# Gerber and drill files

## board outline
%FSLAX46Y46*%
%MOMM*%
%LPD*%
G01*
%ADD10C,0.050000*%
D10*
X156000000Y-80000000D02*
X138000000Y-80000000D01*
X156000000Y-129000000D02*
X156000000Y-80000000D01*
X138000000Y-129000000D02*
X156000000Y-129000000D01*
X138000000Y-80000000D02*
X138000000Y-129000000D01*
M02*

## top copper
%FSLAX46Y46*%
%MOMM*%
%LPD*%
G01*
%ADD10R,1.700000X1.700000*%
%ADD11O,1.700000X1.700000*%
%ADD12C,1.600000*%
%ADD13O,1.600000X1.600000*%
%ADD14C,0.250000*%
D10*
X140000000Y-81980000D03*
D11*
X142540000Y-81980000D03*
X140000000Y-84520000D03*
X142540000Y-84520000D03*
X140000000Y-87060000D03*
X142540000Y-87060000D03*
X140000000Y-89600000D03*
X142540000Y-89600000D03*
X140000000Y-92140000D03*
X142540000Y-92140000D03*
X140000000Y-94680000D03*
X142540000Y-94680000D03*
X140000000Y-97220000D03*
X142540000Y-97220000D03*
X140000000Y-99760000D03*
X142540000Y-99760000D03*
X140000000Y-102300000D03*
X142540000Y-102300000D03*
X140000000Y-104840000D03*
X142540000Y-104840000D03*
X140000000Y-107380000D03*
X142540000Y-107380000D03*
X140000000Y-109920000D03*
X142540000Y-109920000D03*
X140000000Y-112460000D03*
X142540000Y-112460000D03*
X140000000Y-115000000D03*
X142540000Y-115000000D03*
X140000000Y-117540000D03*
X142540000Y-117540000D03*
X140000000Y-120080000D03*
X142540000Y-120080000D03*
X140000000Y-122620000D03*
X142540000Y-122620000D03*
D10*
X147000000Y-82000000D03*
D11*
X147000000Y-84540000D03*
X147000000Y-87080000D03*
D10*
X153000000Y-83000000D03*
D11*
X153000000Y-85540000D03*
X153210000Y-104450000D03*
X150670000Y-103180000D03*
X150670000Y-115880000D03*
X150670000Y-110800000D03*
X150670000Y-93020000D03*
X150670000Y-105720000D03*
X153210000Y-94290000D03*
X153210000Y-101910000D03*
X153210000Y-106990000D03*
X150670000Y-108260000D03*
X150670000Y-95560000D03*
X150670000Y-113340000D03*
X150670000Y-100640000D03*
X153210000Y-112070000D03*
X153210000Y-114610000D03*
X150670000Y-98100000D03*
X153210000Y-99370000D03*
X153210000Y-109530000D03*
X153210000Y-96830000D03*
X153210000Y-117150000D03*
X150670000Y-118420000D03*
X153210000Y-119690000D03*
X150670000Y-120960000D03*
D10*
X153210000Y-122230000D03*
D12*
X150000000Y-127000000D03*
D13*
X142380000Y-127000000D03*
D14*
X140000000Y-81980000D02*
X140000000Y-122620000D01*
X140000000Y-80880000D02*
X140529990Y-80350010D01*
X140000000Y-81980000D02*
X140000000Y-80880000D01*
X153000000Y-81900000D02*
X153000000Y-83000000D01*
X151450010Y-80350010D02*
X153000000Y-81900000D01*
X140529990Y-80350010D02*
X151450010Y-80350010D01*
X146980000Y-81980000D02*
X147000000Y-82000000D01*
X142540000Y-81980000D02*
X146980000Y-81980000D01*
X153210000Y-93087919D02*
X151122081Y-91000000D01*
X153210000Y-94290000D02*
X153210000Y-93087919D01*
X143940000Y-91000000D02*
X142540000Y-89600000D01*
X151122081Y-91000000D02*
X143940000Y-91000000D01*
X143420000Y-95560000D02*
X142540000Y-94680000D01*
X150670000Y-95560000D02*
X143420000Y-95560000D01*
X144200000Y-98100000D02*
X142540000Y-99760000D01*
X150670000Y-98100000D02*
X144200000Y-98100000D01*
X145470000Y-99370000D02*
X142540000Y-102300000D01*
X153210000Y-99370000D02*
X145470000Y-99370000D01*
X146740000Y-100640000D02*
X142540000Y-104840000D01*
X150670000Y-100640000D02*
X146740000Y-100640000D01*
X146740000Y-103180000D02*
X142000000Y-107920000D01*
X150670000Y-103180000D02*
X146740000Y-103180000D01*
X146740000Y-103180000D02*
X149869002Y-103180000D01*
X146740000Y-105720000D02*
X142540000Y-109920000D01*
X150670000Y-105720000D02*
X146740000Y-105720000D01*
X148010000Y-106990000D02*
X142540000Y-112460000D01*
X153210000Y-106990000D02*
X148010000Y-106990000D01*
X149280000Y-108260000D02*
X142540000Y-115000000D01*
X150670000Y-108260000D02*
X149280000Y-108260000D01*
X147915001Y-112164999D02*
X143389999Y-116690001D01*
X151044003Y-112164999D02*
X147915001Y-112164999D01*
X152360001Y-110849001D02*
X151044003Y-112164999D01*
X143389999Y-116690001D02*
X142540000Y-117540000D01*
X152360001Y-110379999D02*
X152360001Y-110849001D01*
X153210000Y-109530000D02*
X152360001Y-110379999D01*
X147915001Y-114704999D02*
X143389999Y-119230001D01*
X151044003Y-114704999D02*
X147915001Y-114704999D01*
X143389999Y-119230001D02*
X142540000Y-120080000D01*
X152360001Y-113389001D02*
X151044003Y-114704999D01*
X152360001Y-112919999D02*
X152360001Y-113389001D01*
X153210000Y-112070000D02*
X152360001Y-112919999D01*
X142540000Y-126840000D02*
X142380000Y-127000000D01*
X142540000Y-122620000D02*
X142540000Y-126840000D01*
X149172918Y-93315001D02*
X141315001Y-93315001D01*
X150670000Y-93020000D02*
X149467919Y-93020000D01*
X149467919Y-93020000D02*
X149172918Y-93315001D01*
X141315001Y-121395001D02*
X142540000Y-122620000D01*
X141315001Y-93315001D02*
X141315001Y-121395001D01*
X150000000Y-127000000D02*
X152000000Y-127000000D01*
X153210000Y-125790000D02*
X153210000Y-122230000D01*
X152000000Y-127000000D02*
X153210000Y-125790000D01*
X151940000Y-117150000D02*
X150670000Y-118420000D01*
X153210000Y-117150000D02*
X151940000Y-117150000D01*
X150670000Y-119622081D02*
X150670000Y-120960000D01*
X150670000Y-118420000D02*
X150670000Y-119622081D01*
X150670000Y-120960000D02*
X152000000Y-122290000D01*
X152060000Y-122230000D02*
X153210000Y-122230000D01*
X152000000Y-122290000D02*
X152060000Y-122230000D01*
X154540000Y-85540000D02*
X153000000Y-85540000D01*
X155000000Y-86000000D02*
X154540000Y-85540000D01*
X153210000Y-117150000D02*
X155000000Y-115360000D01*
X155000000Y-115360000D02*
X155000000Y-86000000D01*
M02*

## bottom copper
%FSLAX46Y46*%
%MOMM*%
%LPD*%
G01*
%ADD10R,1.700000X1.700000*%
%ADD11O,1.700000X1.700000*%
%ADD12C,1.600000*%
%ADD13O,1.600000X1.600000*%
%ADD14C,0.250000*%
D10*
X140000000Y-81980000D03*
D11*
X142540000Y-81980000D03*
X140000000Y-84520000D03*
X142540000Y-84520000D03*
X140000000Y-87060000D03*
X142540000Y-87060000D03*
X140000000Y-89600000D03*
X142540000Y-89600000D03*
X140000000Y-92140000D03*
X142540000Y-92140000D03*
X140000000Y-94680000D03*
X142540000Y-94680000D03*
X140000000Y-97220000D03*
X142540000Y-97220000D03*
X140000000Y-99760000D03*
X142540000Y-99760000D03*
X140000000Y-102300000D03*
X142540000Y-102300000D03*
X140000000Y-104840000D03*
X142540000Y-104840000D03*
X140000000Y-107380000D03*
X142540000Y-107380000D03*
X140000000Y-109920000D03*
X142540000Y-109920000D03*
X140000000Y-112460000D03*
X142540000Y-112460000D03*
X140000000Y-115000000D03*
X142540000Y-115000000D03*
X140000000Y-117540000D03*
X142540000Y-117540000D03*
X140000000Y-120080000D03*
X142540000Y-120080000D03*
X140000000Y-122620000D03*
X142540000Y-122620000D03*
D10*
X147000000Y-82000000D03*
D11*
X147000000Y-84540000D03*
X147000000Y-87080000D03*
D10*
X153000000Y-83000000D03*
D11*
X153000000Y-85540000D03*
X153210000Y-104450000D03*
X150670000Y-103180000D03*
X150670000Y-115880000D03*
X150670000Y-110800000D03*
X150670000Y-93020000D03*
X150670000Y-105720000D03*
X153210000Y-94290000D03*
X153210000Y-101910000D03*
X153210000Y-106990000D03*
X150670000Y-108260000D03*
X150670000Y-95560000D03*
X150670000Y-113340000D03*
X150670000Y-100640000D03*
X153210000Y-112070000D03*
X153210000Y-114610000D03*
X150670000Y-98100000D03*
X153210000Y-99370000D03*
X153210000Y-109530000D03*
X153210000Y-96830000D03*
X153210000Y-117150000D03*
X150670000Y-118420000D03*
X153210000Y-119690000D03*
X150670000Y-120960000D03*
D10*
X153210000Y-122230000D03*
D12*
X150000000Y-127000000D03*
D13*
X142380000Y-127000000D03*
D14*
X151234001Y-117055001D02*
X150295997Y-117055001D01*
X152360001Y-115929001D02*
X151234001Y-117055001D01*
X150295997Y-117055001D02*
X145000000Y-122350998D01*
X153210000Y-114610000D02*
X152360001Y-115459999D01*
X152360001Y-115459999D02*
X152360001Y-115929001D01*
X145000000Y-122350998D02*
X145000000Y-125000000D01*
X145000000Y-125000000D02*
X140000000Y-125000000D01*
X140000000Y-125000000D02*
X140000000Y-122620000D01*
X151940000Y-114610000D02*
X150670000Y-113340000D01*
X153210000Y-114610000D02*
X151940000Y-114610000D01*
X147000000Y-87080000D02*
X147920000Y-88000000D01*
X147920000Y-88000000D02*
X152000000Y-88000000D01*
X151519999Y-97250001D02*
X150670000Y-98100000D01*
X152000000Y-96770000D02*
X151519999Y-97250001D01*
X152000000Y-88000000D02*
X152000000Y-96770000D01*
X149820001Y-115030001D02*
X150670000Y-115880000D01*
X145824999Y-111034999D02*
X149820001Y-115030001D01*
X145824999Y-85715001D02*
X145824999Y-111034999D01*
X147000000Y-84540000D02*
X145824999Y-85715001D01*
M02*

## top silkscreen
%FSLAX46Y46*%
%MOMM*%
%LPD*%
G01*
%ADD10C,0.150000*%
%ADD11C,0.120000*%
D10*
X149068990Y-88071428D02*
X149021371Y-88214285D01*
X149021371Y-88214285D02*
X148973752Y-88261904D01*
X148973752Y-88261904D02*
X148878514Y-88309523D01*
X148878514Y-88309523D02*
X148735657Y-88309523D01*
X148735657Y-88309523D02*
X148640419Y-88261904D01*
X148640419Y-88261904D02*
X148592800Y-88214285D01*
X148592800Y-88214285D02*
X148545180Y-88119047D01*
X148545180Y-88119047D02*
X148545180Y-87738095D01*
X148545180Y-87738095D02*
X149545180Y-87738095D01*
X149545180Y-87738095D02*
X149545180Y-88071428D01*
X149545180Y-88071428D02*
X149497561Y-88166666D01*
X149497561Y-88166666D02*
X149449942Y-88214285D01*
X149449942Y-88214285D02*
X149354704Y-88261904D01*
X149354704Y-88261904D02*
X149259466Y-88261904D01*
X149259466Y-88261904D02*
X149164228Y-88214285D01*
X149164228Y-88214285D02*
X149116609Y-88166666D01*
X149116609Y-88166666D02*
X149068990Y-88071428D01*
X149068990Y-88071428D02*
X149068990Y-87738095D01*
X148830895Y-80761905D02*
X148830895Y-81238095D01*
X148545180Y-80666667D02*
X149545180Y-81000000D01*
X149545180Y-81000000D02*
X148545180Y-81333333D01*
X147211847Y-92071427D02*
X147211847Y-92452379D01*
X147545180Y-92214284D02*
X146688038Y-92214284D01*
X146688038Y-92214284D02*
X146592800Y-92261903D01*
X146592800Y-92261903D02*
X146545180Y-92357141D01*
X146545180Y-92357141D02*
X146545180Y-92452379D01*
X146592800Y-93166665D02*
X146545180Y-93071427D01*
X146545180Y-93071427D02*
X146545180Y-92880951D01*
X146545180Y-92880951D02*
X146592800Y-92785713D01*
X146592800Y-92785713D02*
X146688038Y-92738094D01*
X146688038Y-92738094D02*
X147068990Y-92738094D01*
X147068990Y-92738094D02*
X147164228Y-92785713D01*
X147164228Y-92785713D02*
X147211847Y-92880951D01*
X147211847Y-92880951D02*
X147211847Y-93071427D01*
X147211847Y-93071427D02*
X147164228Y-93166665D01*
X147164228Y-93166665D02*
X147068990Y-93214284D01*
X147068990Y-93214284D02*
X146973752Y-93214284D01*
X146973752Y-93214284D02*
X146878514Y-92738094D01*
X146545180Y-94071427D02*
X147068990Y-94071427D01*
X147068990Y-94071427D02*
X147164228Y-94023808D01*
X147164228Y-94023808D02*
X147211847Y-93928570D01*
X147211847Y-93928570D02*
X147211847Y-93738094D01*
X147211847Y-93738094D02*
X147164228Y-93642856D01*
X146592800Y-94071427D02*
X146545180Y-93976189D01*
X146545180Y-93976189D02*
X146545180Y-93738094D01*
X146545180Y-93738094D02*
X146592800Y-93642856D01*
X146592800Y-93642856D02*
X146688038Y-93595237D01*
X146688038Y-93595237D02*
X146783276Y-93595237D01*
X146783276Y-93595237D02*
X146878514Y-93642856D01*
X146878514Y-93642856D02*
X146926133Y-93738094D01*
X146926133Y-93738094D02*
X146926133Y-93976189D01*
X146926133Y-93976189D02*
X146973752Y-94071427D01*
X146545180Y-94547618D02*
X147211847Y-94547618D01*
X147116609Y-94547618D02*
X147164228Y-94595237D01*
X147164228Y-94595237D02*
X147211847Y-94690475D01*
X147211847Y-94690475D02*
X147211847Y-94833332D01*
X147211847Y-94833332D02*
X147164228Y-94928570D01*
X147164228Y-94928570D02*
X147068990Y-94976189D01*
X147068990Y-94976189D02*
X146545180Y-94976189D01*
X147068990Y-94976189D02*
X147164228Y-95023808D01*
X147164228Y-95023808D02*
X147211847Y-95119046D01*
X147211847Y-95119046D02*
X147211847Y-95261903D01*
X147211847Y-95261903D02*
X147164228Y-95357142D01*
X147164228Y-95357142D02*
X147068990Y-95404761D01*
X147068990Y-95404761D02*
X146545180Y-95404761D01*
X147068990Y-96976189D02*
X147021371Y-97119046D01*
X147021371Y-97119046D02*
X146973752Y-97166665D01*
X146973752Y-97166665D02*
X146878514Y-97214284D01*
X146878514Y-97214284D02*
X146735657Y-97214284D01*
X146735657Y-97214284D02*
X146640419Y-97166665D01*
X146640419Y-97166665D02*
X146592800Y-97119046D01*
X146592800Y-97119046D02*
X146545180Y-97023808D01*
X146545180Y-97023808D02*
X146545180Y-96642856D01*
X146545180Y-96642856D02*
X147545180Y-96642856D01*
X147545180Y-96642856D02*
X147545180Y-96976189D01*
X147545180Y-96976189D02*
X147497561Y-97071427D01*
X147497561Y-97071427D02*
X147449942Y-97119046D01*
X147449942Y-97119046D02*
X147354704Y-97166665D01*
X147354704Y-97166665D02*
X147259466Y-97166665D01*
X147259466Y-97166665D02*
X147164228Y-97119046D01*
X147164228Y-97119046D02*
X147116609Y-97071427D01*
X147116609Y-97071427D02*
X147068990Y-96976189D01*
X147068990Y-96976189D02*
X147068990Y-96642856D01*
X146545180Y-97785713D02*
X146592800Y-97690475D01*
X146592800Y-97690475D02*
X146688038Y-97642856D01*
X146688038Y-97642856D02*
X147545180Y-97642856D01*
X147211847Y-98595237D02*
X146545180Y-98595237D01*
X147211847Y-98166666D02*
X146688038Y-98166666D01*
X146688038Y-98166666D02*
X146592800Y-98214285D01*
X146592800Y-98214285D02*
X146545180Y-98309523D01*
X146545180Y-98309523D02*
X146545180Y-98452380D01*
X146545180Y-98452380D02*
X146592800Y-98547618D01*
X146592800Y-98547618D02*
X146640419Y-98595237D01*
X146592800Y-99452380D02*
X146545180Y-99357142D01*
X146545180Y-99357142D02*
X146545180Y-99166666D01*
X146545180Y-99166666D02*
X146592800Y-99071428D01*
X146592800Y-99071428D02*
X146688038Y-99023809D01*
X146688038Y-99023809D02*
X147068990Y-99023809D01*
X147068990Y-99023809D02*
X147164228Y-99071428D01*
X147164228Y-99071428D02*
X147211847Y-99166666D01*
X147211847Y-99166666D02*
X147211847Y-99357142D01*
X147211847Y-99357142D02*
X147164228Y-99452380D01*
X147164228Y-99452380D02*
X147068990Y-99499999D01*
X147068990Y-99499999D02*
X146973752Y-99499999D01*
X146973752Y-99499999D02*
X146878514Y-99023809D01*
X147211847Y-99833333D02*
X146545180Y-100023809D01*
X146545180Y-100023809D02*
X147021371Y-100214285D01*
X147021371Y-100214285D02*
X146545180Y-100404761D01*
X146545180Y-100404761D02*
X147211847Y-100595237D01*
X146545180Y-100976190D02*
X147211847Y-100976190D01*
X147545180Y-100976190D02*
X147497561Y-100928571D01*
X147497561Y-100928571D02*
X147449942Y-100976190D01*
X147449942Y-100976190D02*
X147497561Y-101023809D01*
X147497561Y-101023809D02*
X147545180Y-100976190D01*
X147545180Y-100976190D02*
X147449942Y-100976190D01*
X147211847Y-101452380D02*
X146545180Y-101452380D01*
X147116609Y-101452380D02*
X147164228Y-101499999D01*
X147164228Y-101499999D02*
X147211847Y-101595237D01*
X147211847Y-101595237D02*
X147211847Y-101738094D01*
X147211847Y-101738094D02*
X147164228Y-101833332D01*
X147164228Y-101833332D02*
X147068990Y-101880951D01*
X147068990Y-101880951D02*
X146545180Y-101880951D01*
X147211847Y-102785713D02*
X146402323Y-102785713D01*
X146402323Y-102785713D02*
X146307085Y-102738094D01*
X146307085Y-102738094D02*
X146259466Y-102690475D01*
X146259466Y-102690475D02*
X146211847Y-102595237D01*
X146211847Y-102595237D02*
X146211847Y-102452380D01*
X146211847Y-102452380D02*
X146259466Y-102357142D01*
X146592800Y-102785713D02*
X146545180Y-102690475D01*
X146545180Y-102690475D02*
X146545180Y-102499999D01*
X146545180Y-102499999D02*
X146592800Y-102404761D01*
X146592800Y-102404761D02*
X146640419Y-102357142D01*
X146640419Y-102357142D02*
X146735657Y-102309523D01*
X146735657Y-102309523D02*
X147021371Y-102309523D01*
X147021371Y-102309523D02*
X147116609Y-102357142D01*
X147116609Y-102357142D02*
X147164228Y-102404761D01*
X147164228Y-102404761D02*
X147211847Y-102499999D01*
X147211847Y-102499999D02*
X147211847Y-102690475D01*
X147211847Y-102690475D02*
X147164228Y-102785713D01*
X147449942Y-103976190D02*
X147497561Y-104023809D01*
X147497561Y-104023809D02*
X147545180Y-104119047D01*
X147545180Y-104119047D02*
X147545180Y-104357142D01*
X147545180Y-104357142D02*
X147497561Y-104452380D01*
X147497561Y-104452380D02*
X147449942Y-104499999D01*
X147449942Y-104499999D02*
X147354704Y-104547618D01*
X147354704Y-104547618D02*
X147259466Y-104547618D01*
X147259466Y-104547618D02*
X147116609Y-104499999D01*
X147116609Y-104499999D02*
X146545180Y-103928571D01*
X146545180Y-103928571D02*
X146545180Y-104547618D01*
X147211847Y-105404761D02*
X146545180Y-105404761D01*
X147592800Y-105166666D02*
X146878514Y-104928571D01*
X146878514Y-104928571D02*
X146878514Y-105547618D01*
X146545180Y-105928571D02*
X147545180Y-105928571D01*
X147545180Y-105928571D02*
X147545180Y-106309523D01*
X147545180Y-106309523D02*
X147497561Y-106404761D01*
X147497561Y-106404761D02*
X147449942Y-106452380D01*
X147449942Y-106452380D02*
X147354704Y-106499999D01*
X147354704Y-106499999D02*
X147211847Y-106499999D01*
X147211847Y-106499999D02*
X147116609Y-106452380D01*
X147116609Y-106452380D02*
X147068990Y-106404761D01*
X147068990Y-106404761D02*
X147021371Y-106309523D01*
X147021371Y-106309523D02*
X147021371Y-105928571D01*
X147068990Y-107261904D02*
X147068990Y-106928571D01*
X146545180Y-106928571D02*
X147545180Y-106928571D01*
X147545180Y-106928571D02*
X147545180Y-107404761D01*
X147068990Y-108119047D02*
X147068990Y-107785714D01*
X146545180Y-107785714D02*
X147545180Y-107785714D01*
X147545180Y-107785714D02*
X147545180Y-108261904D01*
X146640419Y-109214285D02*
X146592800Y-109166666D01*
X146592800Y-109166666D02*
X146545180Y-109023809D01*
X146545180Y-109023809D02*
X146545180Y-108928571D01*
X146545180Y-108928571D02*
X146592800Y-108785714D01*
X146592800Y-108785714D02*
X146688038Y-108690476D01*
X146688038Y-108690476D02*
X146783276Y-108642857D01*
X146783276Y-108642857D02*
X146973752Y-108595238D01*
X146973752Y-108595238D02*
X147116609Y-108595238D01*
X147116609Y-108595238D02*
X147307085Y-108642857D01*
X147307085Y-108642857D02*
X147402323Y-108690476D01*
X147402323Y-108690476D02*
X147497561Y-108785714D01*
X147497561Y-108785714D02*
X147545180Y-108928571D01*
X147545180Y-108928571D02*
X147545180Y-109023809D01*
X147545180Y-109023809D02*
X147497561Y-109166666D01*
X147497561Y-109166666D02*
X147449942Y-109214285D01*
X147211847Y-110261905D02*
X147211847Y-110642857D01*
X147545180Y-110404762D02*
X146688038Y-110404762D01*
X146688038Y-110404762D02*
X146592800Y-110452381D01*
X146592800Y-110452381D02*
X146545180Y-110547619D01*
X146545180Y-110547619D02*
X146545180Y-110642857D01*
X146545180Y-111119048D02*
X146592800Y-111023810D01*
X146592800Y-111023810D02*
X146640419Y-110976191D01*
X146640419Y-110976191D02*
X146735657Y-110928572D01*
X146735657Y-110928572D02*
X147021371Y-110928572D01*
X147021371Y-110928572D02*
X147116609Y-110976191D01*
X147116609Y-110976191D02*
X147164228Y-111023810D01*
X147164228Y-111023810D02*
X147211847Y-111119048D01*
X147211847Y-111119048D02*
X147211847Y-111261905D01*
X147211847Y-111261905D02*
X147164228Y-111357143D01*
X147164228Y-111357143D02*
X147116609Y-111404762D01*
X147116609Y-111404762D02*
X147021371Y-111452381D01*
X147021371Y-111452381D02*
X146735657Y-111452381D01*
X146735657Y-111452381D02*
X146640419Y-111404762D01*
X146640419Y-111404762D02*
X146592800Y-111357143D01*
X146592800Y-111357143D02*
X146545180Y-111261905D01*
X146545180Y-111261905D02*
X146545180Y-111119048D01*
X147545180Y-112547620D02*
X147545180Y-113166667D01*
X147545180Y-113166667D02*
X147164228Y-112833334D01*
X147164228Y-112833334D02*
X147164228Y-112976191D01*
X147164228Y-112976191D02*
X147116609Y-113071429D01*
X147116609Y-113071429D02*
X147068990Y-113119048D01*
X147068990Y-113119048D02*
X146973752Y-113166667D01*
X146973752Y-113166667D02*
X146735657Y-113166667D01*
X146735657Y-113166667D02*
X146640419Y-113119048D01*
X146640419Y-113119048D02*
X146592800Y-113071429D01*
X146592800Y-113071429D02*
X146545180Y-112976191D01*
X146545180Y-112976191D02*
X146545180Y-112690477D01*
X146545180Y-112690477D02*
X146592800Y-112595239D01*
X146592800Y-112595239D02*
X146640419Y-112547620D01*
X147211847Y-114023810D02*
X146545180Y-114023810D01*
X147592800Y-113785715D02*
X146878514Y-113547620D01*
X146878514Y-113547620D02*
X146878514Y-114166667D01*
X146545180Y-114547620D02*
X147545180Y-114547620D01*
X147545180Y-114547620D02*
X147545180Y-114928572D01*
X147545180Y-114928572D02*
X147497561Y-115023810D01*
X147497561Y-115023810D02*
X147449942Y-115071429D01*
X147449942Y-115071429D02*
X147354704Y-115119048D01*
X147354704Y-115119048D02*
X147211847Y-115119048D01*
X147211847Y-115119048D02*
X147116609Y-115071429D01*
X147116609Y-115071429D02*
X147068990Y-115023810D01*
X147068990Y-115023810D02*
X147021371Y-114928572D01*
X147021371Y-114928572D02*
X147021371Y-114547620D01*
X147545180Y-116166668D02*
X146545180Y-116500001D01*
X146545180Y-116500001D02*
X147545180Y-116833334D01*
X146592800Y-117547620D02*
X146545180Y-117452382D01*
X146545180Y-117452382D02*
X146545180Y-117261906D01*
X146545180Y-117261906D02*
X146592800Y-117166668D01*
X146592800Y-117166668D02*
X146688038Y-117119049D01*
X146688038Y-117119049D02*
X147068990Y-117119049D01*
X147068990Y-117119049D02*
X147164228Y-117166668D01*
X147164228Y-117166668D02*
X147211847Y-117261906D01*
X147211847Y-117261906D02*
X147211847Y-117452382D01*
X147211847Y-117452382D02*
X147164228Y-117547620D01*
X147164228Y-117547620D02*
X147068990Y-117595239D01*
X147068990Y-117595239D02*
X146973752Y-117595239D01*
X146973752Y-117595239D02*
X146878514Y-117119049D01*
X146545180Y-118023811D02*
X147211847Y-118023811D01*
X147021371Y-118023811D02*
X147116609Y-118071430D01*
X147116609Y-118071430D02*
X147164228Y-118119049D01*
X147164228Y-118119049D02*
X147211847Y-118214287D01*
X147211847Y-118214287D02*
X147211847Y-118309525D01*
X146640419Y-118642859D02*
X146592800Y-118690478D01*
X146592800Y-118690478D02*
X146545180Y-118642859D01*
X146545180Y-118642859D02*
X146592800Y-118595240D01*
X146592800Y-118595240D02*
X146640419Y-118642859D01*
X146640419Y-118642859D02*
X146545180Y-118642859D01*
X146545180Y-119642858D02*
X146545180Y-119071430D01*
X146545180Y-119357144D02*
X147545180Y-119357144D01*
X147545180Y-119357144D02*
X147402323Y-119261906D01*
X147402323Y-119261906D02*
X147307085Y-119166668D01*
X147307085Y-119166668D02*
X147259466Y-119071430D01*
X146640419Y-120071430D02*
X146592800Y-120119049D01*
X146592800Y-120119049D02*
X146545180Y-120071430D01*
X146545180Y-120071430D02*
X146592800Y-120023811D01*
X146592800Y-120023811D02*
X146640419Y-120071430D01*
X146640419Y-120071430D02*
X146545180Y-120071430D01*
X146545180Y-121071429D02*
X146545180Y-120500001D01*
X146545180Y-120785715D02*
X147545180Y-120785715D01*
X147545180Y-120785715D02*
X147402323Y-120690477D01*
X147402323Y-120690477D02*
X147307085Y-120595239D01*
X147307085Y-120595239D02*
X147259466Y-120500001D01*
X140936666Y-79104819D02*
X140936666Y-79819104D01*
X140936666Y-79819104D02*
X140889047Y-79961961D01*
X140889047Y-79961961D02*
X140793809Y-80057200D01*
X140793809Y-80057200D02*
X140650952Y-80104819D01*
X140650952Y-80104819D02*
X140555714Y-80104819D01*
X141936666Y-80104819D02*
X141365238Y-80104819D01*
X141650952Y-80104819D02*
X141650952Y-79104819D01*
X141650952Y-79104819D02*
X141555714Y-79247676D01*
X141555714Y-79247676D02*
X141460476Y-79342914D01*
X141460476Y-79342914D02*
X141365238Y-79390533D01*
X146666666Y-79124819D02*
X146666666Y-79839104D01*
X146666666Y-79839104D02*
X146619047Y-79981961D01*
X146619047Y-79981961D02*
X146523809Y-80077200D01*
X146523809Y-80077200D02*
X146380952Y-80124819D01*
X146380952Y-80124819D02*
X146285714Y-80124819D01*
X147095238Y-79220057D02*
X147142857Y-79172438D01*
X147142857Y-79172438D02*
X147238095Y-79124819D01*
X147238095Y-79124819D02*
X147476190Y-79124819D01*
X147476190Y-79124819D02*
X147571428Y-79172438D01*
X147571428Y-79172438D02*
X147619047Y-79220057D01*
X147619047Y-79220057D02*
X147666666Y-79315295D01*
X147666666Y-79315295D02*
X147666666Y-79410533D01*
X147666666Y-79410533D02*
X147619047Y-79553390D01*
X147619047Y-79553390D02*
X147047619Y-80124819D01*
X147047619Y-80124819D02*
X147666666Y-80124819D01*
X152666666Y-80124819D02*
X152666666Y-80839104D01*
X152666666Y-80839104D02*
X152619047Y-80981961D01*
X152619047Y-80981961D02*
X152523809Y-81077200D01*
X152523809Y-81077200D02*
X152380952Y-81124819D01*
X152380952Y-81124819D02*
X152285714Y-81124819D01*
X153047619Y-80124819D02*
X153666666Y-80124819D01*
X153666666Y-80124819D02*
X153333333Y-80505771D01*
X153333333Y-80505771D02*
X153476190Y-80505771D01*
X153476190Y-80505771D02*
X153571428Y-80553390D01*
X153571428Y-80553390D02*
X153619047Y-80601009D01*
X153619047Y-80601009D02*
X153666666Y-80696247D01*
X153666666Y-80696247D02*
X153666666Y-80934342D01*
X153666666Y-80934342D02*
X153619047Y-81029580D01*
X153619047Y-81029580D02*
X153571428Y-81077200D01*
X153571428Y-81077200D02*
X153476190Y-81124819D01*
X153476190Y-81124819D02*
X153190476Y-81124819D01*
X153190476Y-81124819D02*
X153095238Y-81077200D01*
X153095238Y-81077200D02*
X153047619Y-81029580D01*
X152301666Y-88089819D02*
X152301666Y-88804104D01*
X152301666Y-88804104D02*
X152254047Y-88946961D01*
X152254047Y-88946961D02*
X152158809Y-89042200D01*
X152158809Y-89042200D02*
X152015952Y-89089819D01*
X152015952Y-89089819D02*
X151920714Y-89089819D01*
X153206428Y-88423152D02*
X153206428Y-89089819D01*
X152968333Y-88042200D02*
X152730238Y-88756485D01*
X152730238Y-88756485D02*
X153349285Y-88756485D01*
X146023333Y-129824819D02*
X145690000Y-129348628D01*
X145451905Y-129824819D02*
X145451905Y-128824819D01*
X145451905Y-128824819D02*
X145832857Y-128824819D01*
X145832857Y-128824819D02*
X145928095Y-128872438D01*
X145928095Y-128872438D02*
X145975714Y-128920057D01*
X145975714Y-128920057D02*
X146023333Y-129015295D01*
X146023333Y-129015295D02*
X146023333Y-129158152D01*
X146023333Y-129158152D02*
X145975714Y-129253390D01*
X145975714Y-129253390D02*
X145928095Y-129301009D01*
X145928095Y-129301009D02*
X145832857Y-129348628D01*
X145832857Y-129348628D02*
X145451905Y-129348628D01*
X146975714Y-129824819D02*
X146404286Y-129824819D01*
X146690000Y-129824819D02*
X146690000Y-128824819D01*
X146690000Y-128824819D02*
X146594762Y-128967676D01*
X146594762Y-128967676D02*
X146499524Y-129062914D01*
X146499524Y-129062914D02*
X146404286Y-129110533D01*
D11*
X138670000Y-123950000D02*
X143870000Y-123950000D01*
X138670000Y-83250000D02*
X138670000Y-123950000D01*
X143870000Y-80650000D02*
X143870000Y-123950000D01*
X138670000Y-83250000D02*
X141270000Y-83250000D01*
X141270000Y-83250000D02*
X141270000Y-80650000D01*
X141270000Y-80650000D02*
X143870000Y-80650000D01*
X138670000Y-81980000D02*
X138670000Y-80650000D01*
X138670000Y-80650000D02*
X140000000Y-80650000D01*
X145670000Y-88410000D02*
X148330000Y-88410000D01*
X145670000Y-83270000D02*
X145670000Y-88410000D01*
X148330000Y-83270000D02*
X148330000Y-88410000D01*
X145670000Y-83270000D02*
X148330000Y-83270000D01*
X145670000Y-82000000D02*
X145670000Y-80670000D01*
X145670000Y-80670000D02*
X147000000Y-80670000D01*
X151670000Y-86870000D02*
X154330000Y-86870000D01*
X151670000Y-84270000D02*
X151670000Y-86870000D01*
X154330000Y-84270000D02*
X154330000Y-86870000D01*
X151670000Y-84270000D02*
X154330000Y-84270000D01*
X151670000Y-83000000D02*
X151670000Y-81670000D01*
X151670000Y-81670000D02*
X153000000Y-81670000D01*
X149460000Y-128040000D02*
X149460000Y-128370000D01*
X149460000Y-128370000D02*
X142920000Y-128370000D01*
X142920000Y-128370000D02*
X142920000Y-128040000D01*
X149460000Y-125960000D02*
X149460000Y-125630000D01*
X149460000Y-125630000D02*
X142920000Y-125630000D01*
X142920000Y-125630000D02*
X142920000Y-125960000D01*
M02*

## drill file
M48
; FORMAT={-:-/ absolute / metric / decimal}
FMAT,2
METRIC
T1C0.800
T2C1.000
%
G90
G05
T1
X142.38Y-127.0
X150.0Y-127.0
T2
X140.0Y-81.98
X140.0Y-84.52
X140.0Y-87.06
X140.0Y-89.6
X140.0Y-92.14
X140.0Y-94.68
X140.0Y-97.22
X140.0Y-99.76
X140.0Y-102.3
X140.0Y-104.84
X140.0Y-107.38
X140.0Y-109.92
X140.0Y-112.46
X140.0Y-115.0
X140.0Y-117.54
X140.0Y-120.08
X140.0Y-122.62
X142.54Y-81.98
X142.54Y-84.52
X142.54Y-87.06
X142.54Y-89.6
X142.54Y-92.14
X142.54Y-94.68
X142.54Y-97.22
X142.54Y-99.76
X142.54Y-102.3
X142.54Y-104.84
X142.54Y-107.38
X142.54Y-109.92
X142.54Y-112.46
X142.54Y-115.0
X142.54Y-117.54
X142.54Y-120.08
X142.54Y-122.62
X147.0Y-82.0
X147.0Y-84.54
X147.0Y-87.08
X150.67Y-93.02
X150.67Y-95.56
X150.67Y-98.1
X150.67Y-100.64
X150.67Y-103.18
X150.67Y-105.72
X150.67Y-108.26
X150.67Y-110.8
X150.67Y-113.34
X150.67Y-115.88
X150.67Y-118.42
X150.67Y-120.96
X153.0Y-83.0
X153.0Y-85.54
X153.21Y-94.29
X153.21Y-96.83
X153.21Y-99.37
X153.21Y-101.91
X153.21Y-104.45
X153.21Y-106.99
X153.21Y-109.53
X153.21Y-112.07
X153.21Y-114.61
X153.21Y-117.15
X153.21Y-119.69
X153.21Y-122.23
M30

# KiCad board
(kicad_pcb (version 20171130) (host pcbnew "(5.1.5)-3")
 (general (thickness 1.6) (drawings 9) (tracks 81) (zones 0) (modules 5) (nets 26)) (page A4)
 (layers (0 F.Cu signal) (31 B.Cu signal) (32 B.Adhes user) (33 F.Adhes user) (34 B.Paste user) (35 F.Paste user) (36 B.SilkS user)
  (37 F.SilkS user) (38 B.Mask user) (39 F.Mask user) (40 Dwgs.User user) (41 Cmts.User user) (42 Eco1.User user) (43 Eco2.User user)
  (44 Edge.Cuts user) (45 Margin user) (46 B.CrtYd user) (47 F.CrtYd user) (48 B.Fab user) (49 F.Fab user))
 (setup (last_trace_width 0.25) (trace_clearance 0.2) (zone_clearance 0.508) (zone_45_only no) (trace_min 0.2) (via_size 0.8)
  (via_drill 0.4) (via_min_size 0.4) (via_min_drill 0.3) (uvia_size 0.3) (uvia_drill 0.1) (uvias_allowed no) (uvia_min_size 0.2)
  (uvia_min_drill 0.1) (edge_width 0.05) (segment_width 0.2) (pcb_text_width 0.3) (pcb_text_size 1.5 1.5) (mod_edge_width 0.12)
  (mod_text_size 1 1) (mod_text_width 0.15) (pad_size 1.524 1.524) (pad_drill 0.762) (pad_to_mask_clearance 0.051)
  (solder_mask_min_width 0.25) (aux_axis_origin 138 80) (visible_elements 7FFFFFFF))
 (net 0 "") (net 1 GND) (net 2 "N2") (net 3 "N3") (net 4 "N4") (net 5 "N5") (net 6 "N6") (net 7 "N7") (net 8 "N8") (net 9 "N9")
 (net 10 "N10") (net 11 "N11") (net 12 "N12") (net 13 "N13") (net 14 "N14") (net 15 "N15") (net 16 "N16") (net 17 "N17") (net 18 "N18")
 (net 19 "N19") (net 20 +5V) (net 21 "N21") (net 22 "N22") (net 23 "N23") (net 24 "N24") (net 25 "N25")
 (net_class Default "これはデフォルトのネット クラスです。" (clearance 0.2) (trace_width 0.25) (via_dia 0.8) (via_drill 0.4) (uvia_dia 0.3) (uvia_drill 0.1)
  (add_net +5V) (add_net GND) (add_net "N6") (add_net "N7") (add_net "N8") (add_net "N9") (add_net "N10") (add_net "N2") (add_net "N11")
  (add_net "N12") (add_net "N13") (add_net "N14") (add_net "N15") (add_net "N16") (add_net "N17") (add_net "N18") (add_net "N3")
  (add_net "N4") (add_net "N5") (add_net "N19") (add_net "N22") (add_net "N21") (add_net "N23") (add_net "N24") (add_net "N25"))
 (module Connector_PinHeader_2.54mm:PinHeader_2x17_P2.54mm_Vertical (layer F.Cu) (at 140 81.98)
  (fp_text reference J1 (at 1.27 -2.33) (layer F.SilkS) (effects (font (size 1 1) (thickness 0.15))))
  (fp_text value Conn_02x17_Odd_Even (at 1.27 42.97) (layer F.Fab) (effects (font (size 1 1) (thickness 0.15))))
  (fp_line (start -1.33 41.97) (end 3.87 41.97) (layer F.SilkS) (width 0.12))
  (fp_line (start -1.33 1.27) (end -1.33 41.97) (layer F.SilkS) (width 0.12))
  (fp_line (start 3.87 -1.33) (end 3.87 41.97) (layer F.SilkS) (width 0.12))
  (fp_line (start -1.33 1.27) (end 1.27 1.27) (layer F.SilkS) (width 0.12))
  (fp_line (start 1.27 1.27) (end 1.27 -1.33) (layer F.SilkS) (width 0.12))
  (fp_line (start 1.27 -1.33) (end 3.87 -1.33) (layer F.SilkS) (width 0.12))
  (fp_line (start -1.33 0) (end -1.33 -1.33) (layer F.SilkS) (width 0.12))
  (fp_line (start -1.33 -1.33) (end 0 -1.33) (layer F.SilkS) (width 0.12))
  (pad 1 thru_hole rect (at 0 0) (size 1.7 1.7) (drill 1) (layers *.Cu *.Mask) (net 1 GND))
  (pad 2 thru_hole oval (at 2.54 0) (size 1.7 1.7) (drill 1) (layers *.Cu *.Mask) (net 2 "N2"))
  (pad 3 thru_hole oval (at 0 2.54) (size 1.7 1.7) (drill 1) (layers *.Cu *.Mask) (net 1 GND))
  (pad 4 thru_hole oval (at 2.54 2.54) (size 1.7 1.7) (drill 1) (layers *.Cu *.Mask) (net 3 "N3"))
  (pad 5 thru_hole oval (at 0 5.08) (size 1.7 1.7) (drill 1) (layers *.Cu *.Mask) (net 1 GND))
  (pad 6 thru_hole oval (at 2.54 5.08) (size 1.7 1.7) (drill 1) (layers *.Cu *.Mask) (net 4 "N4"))
  (pad 7 thru_hole oval (at 0 7.62) (size 1.7 1.7) (drill 1) (layers *.Cu *.Mask) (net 1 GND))
  (pad 8 thru_hole oval (at 2.54 7.62) (size 1.7 1.7) (drill 1) (layers *.Cu *.Mask) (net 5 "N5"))
  (pad 9 thru_hole oval (at 0 10.16) (size 1.7 1.7) (drill 1) (layers *.Cu *.Mask) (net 1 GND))
  (pad 10 thru_hole oval (at 2.54 10.16) (size 1.7 1.7) (drill 1) (layers *.Cu *.Mask) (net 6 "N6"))
  (pad 11 thru_hole oval (at 0 12.7) (size 1.7 1.7) (drill 1) (layers *.Cu *.Mask) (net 1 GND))
  (pad 12 thru_hole oval (at 2.54 12.7) (size 1.7 1.7) (drill 1) (layers *.Cu *.Mask) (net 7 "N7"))
  (pad 13 thru_hole oval (at 0 15.24) (size 1.7 1.7) (drill 1) (layers *.Cu *.Mask) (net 1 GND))
  (pad 14 thru_hole oval (at 2.54 15.24) (size 1.7 1.7) (drill 1) (layers *.Cu *.Mask) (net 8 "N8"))
  (pad 15 thru_hole oval (at 0 17.78) (size 1.7 1.7) (drill 1) (layers *.Cu *.Mask) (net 1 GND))
  (pad 16 thru_hole oval (at 2.54 17.78) (size 1.7 1.7) (drill 1) (layers *.Cu *.Mask) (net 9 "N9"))
  (pad 17 thru_hole oval (at 0 20.32) (size 1.7 1.7) (drill 1) (layers *.Cu *.Mask) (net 1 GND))
  (pad 18 thru_hole oval (at 2.54 20.32) (size 1.7 1.7) (drill 1) (layers *.Cu *.Mask) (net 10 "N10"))
  (pad 19 thru_hole oval (at 0 22.86) (size 1.7 1.7) (drill 1) (layers *.Cu *.Mask) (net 1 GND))
  (pad 20 thru_hole oval (at 2.54 22.86) (size 1.7 1.7) (drill 1) (layers *.Cu *.Mask) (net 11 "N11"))
  (pad 21 thru_hole oval (at 0 25.4) (size 1.7 1.7) (drill 1) (layers *.Cu *.Mask) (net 1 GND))
  (pad 22 thru_hole oval (at 2.54 25.4) (size 1.7 1.7) (drill 1) (layers *.Cu *.Mask) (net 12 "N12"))
  (pad 23 thru_hole oval (at 0 27.94) (size 1.7 1.7) (drill 1) (layers *.Cu *.Mask) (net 1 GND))
  (pad 24 thru_hole oval (at 2.54 27.94) (size 1.7 1.7) (drill 1) (layers *.Cu *.Mask) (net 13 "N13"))
  (pad 25 thru_hole oval (at 0 30.48) (size 1.7 1.7) (drill 1) (layers *.Cu *.Mask) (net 1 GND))
  (pad 26 thru_hole oval (at 2.54 30.48) (size 1.7 1.7) (drill 1) (layers *.Cu *.Mask) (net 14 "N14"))
  (pad 27 thru_hole oval (at 0 33.02) (size 1.7 1.7) (drill 1) (layers *.Cu *.Mask) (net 1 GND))
  (pad 28 thru_hole oval (at 2.54 33.02) (size 1.7 1.7) (drill 1) (layers *.Cu *.Mask) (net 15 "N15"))
  (pad 29 thru_hole oval (at 0 35.56) (size 1.7 1.7) (drill 1) (layers *.Cu *.Mask) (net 1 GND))
  (pad 30 thru_hole oval (at 2.54 35.56) (size 1.7 1.7) (drill 1) (layers *.Cu *.Mask) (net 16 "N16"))
  (pad 31 thru_hole oval (at 0 38.1) (size 1.7 1.7) (drill 1) (layers *.Cu *.Mask) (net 1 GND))
  (pad 32 thru_hole oval (at 2.54 38.1) (size 1.7 1.7) (drill 1) (layers *.Cu *.Mask) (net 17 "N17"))
  (pad 33 thru_hole oval (at 0 40.64) (size 1.7 1.7) (drill 1) (layers *.Cu *.Mask) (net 1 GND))
  (pad 34 thru_hole oval (at 2.54 40.64) (size 1.7 1.7) (drill 1) (layers *.Cu *.Mask) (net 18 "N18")))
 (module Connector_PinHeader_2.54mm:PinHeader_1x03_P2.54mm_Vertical (layer F.Cu) (at 147 82)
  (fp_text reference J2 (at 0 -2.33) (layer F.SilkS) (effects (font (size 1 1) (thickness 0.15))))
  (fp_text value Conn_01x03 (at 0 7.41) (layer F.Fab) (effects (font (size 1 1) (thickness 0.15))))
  (fp_line (start -1.33 6.41) (end 1.33 6.41) (layer F.SilkS) (width 0.12))
  (fp_line (start -1.33 1.27) (end -1.33 6.41) (layer F.SilkS) (width 0.12))
  (fp_line (start 1.33 1.27) (end 1.33 6.41) (layer F.SilkS) (width 0.12))
  (fp_line (start -1.33 1.27) (end 1.33 1.27) (layer F.SilkS) (width 0.12))
  (fp_line (start -1.33 0) (end -1.33 -1.33) (layer F.SilkS) (width 0.12))
  (fp_line (start -1.33 -1.33) (end 0 -1.33) (layer F.SilkS) (width 0.12))
  (pad 1 thru_hole rect (at 0 0) (size 1.7 1.7) (drill 1) (layers *.Cu *.Mask) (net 2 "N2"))
  (pad 2 thru_hole oval (at 0 2.54) (size 1.7 1.7) (drill 1) (layers *.Cu *.Mask) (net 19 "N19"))
  (pad 3 thru_hole oval (at 0 5.08) (size 1.7 1.7) (drill 1) (layers *.Cu *.Mask) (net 9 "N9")))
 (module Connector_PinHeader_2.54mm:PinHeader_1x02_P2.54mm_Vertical (layer F.Cu) (at 153 83)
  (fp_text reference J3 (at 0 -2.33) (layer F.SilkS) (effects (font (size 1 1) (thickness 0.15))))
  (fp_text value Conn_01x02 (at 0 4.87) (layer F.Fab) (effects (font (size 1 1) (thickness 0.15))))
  (fp_line (start -1.33 3.87) (end 1.33 3.87) (layer F.SilkS) (width 0.12))
  (fp_line (start -1.33 1.27) (end -1.33 3.87) (layer F.SilkS) (width 0.12))
  (fp_line (start 1.33 1.27) (end 1.33 3.87) (layer F.SilkS) (width 0.12))
  (fp_line (start -1.33 1.27) (end 1.33 1.27) (layer F.SilkS) (width 0.12))
  (fp_line (start -1.33 0) (end -1.33 -1.33) (layer F.SilkS) (width 0.12))
  (fp_line (start -1.33 -1.33) (end 0 -1.33) (layer F.SilkS) (width 0.12))
  (pad 1 thru_hole rect (at 0 0) (size 1.7 1.7) (drill 1) (layers *.Cu *.Mask) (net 1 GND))
  (pad 2 thru_hole oval (at 0 2.54) (size 1.7 1.7) (drill 1) (layers *.Cu *.Mask) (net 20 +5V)))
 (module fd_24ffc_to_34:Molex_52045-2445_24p (layer F.Cu) (at 152 88)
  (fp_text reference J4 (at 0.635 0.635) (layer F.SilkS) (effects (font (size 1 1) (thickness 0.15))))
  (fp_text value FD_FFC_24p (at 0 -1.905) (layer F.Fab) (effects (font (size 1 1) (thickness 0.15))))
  (pad 15 thru_hole oval (at 1.21 16.45) (size 1.7 1.7) (drill 1) (layers *.Cu *.Mask) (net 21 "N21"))
  (pad 16 thru_hole oval (at -1.33 15.18) (size 1.7 1.7) (drill 1) (layers *.Cu *.Mask) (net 12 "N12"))
  (pad 6 thru_hole oval (at -1.33 27.88) (size 1.7 1.7) (drill 1) (layers *.Cu *.Mask) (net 19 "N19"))
  (pad 10 thru_hole oval (at -1.33 22.8) (size 1.7 1.7) (drill 1) (layers *.Cu *.Mask) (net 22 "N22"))
  (pad 24 thru_hole oval (at -1.33 5.02) (size 1.7 1.7) (drill 1) (layers *.Cu *.Mask) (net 18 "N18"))
  (pad 14 thru_hole oval (at -1.33 17.72) (size 1.7 1.7) (drill 1) (layers *.Cu *.Mask) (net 13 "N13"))
  (pad 23 thru_hole oval (at 1.21 6.29) (size 1.7 1.7) (drill 1) (layers *.Cu *.Mask) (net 5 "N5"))
  (pad 17 thru_hole oval (at 1.21 13.91) (size 1.7 1.7) (drill 1) (layers *.Cu *.Mask) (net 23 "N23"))
  (pad 13 thru_hole oval (at 1.21 18.99) (size 1.7 1.7) (drill 1) (layers *.Cu *.Mask) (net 14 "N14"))
  (pad 12 thru_hole oval (at -1.33 20.26) (size 1.7 1.7) (drill 1) (layers *.Cu *.Mask) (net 15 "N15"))
  (pad 22 thru_hole oval (at -1.33 7.56) (size 1.7 1.7) (drill 1) (layers *.Cu *.Mask) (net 7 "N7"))
  (pad 8 thru_hole oval (at -1.33 25.34) (size 1.7 1.7) (drill 1) (layers *.Cu *.Mask) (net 1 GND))
  (pad 18 thru_hole oval (at -1.33 12.64) (size 1.7 1.7) (drill 1) (layers *.Cu *.Mask) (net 11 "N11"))
  (pad 9 thru_hole oval (at 1.21 24.07) (size 1.7 1.7) (drill 1) (layers *.Cu *.Mask) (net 17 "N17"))
  (pad 7 thru_hole oval (at 1.21 26.61) (size 1.7 1.7) (drill 1) (layers *.Cu *.Mask) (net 1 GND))
  (pad 20 thru_hole oval (at -1.33 10.1) (size 1.7 1.7) (drill 1) (layers *.Cu *.Mask) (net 9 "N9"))
  (pad 19 thru_hole oval (at 1.21 11.37) (size 1.7 1.7) (drill 1) (layers *.Cu *.Mask) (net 10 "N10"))
  (pad 11 thru_hole oval (at 1.21 21.53) (size 1.7 1.7) (drill 1) (layers *.Cu *.Mask) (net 16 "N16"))
  (pad 21 thru_hole oval (at 1.21 8.83) (size 1.7 1.7) (drill 1) (layers *.Cu *.Mask) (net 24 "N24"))
  (pad 5 thru_hole oval (at 1.21 29.15) (size 1.7 1.7) (drill 1) (layers *.Cu *.Mask) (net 20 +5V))
  (pad 4 thru_hole oval (at -1.33 30.42) (size 1.7 1.7) (drill 1) (layers *.Cu *.Mask) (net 20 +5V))
  (pad 3 thru_hole oval (at 1.21 31.69) (size 1.7 1.7) (drill 1) (layers *.Cu *.Mask) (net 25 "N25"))
  (pad 2 thru_hole oval (at -1.33 32.96) (size 1.7 1.7) (drill 1) (layers *.Cu *.Mask) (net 20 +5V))
  (pad 1 thru_hole rect (at 1.21 34.23) (size 1.7 1.7) (drill 1) (layers *.Cu *.Mask) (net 20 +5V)))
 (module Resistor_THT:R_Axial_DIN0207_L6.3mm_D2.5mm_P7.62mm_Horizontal (layer F.Cu) (at 150 127 180)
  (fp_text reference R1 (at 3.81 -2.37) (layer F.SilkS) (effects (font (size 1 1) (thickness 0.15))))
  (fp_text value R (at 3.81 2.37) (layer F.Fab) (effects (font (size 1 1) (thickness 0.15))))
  (fp_line (start 0.54 -1.04) (end 0.54 -1.37) (layer F.SilkS) (width 0.12))
  (fp_line (start 0.54 -1.37) (end 7.08 -1.37) (layer F.SilkS) (width 0.12))
  (fp_line (start 7.08 -1.37) (end 7.08 -1.04) (layer F.SilkS) (width 0.12))
  (fp_line (start 0.54 1.04) (end 0.54 1.37) (layer F.SilkS) (width 0.12))
  (fp_line (start 0.54 1.37) (end 7.08 1.37) (layer F.SilkS) (width 0.12))
  (fp_line (start 7.08 1.37) (end 7.08 1.04) (layer F.SilkS) (width 0.12))
  (pad 1 thru_hole circle (at 0 0 180) (size 1.6 1.6) (drill 0.8) (layers *.Cu *.Mask) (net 20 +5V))
  (pad 2 thru_hole oval (at 7.62 0 180) (size 1.6 1.6) (drill 0.8) (layers *.Cu *.Mask) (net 18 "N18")))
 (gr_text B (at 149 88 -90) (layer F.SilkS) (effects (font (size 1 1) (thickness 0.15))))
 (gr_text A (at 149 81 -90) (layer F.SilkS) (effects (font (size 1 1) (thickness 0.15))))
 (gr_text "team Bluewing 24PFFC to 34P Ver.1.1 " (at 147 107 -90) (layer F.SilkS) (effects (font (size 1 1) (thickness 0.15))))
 (gr_line (start 156 80) (end 138 80) (layer Edge.Cuts) (width 0.05))
 (gr_line (start 156 129) (end 156 80) (layer Edge.Cuts) (width 0.05))
 (gr_line (start 138 129) (end 156 129) (layer Edge.Cuts) (width 0.05))
 (gr_line (start 138 80) (end 138 129) (layer Edge.Cuts) (width 0.05))
 (segment (start 140 81.98) (end 140 122.62) (width 0.25) (layer F.Cu) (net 1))
 (segment (start 151.234001 117.055001) (end 150.295997 117.055001) (width 0.25) (layer B.Cu) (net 1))
 (segment (start 152.360001 115.929001) (end 151.234001 117.055001) (width 0.25) (layer B.Cu) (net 1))
 (segment (start 150.295997 117.055001) (end 145 122.350998) (width 0.25) (layer B.Cu) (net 1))
 (segment (start 153.21 114.61) (end 152.360001 115.459999) (width 0.25) (layer B.Cu) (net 1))
 (segment (start 152.360001 115.459999) (end 152.360001 115.929001) (width 0.25) (layer B.Cu) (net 1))
 (segment (start 145 122.350998) (end 145 125) (width 0.25) (layer B.Cu) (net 1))
 (segment (start 145 125) (end 140 125) (width 0.25) (layer B.Cu) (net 1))
 (segment (start 140 125) (end 140 122.62) (width 0.25) (layer B.Cu) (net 1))
 (segment (start 151.94 114.61) (end 150.67 113.34) (width 0.25) (layer B.Cu) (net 1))
 (segment (start 153.21 114.61) (end 151.94 114.61) (width 0.25) (layer B.Cu) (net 1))
 (segment (start 140 80.88) (end 140.52999 80.35001) (width 0.25) (layer F.Cu) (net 1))
 (segment (start 140 81.98) (end 140 80.88) (width 0.25) (layer F.Cu) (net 1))
 (segment (start 153 81.9) (end 153 83) (width 0.25) (layer F.Cu) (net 1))
 (segment (start 151.45001 80.35001) (end 153 81.9) (width 0.25) (layer F.Cu) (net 1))
 (segment (start 140.52999 80.35001) (end 151.45001 80.35001) (width 0.25) (layer F.Cu) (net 1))
 (segment (start 146.98 81.98) (end 147 82) (width 0.25) (layer F.Cu) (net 2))
 (segment (start 142.54 81.98) (end 146.98 81.98) (width 0.25) (layer F.Cu) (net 2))
 (segment (start 153.21 93.087919) (end 151.122081 91) (width 0.25) (layer F.Cu) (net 5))
 (segment (start 153.21 94.29) (end 153.21 93.087919) (width 0.25) (layer F.Cu) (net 5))
 (segment (start 143.94 91) (end 142.54 89.6) (width 0.25) (layer F.Cu) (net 5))
 (segment (start 151.122081 91) (end 143.94 91) (width 0.25) (layer F.Cu) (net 5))
 (segment (start 143.42 95.56) (end 142.54 94.68) (width 0.25) (layer F.Cu) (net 7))
 (segment (start 150.67 95.56) (end 143.42 95.56) (width 0.25) (layer F.Cu) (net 7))
 (segment (start 144.2 98.1) (end 142.54 99.76) (width 0.25) (layer F.Cu) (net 9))
 (segment (start 150.67 98.1) (end 144.2 98.1) (width 0.25) (layer F.Cu) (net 9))
 (segment (start 147 87.08) (end 147.92 88) (width 0.25) (layer B.Cu) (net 9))
 (segment (start 147.92 88) (end 152 88) (width 0.25) (layer B.Cu) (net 9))
 (segment (start 151.519999 97.250001) (end 150.67 98.1) (width 0.25) (layer B.Cu) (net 9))
 (segment (start 152 96.77) (end 151.519999 97.250001) (width 0.25) (layer B.Cu) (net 9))
 (segment (start 152 88) (end 152 96.77) (width 0.25) (layer B.Cu) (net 9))
 (segment (start 145.47 99.37) (end 142.54 102.3) (width 0.25) (layer F.Cu) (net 10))
 (segment (start 153.21 99.37) (end 145.47 99.37) (width 0.25) (layer F.Cu) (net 10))
 (segment (start 146.74 100.64) (end 142.54 104.84) (width 0.25) (layer F.Cu) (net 11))
 (segment (start 150.67 100.64) (end 146.74 100.64) (width 0.25) (layer F.Cu) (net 11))
 (segment (start 146.74 103.18) (end 142 107.92) (width 0.25) (layer F.Cu) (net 12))
 (segment (start 150.67 103.18) (end 146.74 103.18) (width 0.25) (layer F.Cu) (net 12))
 (segment (start 146.74 103.18) (end 149.869002 103.18) (width 0.25) (layer F.Cu) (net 12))
 (segment (start 146.74 105.72) (end 142.54 109.92) (width 0.25) (layer F.Cu) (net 13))
 (segment (start 150.67 105.72) (end 146.74 105.72) (width 0.25) (layer F.Cu) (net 13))
 (segment (start 148.01 106.99) (end 142.54 112.46) (width 0.25) (layer F.Cu) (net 14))
 (segment (start 153.21 106.99) (end 148.01 106.99) (width 0.25) (layer F.Cu) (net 14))
 (segment (start 149.28 108.26) (end 142.54 115) (width 0.25) (layer F.Cu) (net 15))
 (segment (start 150.67 108.26) (end 149.28 108.26) (width 0.25) (layer F.Cu) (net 15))
 (segment (start 147.915001 112.164999) (end 143.389999 116.690001) (width 0.25) (layer F.Cu) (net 16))
 (segment (start 151.044003 112.164999) (end 147.915001 112.164999) (width 0.25) (layer F.Cu) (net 16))
 (segment (start 152.360001 110.849001) (end 151.044003 112.164999) (width 0.25) (layer F.Cu) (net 16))
 (segment (start 143.389999 116.690001) (end 142.54 117.54) (width 0.25) (layer F.Cu) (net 16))
 (segment (start 152.360001 110.379999) (end 152.360001 110.849001) (width 0.25) (layer F.Cu) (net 16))
 (segment (start 153.21 109.53) (end 152.360001 110.379999) (width 0.25) (layer F.Cu) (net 16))
 (segment (start 147.915001 114.704999) (end 143.389999 119.230001) (width 0.25) (layer F.Cu) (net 17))
 (segment (start 151.044003 114.704999) (end 147.915001 114.704999) (width 0.25) (layer F.Cu) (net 17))
 (segment (start 143.389999 119.230001) (end 142.54 120.08) (width 0.25) (layer F.Cu) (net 17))
 (segment (start 152.360001 113.389001) (end 151.044003 114.704999) (width 0.25) (layer F.Cu) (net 17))
 (segment (start 152.360001 112.919999) (end 152.360001 113.389001) (width 0.25) (layer F.Cu) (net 17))
 (segment (start 153.21 112.07) (end 152.360001 112.919999) (width 0.25) (layer F.Cu) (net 17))
 (segment (start 142.54 126.84) (end 142.38 127) (width 0.25) (layer F.Cu) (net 18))
 (segment (start 142.54 122.62) (end 142.54 126.84) (width 0.25) (layer F.Cu) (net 18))
 (segment (start 149.172918 93.315001) (end 141.315001 93.315001) (width 0.25) (layer F.Cu) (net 18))
 (segment (start 150.67 93.02) (end 149.467919 93.02) (width 0.25) (layer F.Cu) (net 18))
 (segment (start 149.467919 93.02) (end 149.172918 93.315001) (width 0.25) (layer F.Cu) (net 18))
 (segment (start 141.315001 121.395001) (end 142.54 122.62) (width 0.25) (layer F.Cu) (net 18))
 (segment (start 141.315001 93.315001) (end 141.315001 121.395001) (width 0.25) (layer F.Cu) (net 18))
 (segment (start 149.820001 115.030001) (end 150.67 115.88) (width 0.25) (layer B.Cu) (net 19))
 (segment (start 145.824999 111.034999) (end 149.820001 115.030001) (width 0.25) (layer B.Cu) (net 19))
 (segment (start 145.824999 85.715001) (end 145.824999 111.034999) (width 0.25) (layer B.Cu) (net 19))
 (segment (start 147 84.54) (end 145.824999 85.715001) (width 0.25) (layer B.Cu) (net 19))
 (segment (start 150 127) (end 152 127) (width 0.25) (layer F.Cu) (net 20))
 (segment (start 153.21 125.79) (end 153.21 122.23) (width 0.25) (layer F.Cu) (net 20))
 (segment (start 152 127) (end 153.21 125.79) (width 0.25) (layer F.Cu) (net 20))
 (segment (start 151.94 117.15) (end 150.67 118.42) (width 0.25) (layer F.Cu) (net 20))
 (segment (start 153.21 117.15) (end 151.94 117.15) (width 0.25) (layer F.Cu) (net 20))
 (segment (start 150.67 119.622081) (end 150.67 120.96) (width 0.25) (layer F.Cu) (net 20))
 (segment (start 150.67 118.42) (end 150.67 119.622081) (width 0.25) (layer F.Cu) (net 20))
 (segment (start 150.67 120.96) (end 152 122.29) (width 0.25) (layer F.Cu) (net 20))
 (segment (start 152.06 122.23) (end 153.21 122.23) (width 0.25) (layer F.Cu) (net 20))
 (segment (start 152 122.29) (end 152.06 122.23) (width 0.25) (layer F.Cu) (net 20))
 (segment (start 154.54 85.54) (end 153 85.54) (width 0.25) (layer F.Cu) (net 20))
 (segment (start 155 86) (end 154.54 85.54) (width 0.25) (layer F.Cu) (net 20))
 (segment (start 153.21 117.15) (end 155 115.36) (width 0.25) (layer F.Cu) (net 20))
 (segment (start 155 115.36) (end 155 86) (width 0.25) (layer F.Cu) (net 20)))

